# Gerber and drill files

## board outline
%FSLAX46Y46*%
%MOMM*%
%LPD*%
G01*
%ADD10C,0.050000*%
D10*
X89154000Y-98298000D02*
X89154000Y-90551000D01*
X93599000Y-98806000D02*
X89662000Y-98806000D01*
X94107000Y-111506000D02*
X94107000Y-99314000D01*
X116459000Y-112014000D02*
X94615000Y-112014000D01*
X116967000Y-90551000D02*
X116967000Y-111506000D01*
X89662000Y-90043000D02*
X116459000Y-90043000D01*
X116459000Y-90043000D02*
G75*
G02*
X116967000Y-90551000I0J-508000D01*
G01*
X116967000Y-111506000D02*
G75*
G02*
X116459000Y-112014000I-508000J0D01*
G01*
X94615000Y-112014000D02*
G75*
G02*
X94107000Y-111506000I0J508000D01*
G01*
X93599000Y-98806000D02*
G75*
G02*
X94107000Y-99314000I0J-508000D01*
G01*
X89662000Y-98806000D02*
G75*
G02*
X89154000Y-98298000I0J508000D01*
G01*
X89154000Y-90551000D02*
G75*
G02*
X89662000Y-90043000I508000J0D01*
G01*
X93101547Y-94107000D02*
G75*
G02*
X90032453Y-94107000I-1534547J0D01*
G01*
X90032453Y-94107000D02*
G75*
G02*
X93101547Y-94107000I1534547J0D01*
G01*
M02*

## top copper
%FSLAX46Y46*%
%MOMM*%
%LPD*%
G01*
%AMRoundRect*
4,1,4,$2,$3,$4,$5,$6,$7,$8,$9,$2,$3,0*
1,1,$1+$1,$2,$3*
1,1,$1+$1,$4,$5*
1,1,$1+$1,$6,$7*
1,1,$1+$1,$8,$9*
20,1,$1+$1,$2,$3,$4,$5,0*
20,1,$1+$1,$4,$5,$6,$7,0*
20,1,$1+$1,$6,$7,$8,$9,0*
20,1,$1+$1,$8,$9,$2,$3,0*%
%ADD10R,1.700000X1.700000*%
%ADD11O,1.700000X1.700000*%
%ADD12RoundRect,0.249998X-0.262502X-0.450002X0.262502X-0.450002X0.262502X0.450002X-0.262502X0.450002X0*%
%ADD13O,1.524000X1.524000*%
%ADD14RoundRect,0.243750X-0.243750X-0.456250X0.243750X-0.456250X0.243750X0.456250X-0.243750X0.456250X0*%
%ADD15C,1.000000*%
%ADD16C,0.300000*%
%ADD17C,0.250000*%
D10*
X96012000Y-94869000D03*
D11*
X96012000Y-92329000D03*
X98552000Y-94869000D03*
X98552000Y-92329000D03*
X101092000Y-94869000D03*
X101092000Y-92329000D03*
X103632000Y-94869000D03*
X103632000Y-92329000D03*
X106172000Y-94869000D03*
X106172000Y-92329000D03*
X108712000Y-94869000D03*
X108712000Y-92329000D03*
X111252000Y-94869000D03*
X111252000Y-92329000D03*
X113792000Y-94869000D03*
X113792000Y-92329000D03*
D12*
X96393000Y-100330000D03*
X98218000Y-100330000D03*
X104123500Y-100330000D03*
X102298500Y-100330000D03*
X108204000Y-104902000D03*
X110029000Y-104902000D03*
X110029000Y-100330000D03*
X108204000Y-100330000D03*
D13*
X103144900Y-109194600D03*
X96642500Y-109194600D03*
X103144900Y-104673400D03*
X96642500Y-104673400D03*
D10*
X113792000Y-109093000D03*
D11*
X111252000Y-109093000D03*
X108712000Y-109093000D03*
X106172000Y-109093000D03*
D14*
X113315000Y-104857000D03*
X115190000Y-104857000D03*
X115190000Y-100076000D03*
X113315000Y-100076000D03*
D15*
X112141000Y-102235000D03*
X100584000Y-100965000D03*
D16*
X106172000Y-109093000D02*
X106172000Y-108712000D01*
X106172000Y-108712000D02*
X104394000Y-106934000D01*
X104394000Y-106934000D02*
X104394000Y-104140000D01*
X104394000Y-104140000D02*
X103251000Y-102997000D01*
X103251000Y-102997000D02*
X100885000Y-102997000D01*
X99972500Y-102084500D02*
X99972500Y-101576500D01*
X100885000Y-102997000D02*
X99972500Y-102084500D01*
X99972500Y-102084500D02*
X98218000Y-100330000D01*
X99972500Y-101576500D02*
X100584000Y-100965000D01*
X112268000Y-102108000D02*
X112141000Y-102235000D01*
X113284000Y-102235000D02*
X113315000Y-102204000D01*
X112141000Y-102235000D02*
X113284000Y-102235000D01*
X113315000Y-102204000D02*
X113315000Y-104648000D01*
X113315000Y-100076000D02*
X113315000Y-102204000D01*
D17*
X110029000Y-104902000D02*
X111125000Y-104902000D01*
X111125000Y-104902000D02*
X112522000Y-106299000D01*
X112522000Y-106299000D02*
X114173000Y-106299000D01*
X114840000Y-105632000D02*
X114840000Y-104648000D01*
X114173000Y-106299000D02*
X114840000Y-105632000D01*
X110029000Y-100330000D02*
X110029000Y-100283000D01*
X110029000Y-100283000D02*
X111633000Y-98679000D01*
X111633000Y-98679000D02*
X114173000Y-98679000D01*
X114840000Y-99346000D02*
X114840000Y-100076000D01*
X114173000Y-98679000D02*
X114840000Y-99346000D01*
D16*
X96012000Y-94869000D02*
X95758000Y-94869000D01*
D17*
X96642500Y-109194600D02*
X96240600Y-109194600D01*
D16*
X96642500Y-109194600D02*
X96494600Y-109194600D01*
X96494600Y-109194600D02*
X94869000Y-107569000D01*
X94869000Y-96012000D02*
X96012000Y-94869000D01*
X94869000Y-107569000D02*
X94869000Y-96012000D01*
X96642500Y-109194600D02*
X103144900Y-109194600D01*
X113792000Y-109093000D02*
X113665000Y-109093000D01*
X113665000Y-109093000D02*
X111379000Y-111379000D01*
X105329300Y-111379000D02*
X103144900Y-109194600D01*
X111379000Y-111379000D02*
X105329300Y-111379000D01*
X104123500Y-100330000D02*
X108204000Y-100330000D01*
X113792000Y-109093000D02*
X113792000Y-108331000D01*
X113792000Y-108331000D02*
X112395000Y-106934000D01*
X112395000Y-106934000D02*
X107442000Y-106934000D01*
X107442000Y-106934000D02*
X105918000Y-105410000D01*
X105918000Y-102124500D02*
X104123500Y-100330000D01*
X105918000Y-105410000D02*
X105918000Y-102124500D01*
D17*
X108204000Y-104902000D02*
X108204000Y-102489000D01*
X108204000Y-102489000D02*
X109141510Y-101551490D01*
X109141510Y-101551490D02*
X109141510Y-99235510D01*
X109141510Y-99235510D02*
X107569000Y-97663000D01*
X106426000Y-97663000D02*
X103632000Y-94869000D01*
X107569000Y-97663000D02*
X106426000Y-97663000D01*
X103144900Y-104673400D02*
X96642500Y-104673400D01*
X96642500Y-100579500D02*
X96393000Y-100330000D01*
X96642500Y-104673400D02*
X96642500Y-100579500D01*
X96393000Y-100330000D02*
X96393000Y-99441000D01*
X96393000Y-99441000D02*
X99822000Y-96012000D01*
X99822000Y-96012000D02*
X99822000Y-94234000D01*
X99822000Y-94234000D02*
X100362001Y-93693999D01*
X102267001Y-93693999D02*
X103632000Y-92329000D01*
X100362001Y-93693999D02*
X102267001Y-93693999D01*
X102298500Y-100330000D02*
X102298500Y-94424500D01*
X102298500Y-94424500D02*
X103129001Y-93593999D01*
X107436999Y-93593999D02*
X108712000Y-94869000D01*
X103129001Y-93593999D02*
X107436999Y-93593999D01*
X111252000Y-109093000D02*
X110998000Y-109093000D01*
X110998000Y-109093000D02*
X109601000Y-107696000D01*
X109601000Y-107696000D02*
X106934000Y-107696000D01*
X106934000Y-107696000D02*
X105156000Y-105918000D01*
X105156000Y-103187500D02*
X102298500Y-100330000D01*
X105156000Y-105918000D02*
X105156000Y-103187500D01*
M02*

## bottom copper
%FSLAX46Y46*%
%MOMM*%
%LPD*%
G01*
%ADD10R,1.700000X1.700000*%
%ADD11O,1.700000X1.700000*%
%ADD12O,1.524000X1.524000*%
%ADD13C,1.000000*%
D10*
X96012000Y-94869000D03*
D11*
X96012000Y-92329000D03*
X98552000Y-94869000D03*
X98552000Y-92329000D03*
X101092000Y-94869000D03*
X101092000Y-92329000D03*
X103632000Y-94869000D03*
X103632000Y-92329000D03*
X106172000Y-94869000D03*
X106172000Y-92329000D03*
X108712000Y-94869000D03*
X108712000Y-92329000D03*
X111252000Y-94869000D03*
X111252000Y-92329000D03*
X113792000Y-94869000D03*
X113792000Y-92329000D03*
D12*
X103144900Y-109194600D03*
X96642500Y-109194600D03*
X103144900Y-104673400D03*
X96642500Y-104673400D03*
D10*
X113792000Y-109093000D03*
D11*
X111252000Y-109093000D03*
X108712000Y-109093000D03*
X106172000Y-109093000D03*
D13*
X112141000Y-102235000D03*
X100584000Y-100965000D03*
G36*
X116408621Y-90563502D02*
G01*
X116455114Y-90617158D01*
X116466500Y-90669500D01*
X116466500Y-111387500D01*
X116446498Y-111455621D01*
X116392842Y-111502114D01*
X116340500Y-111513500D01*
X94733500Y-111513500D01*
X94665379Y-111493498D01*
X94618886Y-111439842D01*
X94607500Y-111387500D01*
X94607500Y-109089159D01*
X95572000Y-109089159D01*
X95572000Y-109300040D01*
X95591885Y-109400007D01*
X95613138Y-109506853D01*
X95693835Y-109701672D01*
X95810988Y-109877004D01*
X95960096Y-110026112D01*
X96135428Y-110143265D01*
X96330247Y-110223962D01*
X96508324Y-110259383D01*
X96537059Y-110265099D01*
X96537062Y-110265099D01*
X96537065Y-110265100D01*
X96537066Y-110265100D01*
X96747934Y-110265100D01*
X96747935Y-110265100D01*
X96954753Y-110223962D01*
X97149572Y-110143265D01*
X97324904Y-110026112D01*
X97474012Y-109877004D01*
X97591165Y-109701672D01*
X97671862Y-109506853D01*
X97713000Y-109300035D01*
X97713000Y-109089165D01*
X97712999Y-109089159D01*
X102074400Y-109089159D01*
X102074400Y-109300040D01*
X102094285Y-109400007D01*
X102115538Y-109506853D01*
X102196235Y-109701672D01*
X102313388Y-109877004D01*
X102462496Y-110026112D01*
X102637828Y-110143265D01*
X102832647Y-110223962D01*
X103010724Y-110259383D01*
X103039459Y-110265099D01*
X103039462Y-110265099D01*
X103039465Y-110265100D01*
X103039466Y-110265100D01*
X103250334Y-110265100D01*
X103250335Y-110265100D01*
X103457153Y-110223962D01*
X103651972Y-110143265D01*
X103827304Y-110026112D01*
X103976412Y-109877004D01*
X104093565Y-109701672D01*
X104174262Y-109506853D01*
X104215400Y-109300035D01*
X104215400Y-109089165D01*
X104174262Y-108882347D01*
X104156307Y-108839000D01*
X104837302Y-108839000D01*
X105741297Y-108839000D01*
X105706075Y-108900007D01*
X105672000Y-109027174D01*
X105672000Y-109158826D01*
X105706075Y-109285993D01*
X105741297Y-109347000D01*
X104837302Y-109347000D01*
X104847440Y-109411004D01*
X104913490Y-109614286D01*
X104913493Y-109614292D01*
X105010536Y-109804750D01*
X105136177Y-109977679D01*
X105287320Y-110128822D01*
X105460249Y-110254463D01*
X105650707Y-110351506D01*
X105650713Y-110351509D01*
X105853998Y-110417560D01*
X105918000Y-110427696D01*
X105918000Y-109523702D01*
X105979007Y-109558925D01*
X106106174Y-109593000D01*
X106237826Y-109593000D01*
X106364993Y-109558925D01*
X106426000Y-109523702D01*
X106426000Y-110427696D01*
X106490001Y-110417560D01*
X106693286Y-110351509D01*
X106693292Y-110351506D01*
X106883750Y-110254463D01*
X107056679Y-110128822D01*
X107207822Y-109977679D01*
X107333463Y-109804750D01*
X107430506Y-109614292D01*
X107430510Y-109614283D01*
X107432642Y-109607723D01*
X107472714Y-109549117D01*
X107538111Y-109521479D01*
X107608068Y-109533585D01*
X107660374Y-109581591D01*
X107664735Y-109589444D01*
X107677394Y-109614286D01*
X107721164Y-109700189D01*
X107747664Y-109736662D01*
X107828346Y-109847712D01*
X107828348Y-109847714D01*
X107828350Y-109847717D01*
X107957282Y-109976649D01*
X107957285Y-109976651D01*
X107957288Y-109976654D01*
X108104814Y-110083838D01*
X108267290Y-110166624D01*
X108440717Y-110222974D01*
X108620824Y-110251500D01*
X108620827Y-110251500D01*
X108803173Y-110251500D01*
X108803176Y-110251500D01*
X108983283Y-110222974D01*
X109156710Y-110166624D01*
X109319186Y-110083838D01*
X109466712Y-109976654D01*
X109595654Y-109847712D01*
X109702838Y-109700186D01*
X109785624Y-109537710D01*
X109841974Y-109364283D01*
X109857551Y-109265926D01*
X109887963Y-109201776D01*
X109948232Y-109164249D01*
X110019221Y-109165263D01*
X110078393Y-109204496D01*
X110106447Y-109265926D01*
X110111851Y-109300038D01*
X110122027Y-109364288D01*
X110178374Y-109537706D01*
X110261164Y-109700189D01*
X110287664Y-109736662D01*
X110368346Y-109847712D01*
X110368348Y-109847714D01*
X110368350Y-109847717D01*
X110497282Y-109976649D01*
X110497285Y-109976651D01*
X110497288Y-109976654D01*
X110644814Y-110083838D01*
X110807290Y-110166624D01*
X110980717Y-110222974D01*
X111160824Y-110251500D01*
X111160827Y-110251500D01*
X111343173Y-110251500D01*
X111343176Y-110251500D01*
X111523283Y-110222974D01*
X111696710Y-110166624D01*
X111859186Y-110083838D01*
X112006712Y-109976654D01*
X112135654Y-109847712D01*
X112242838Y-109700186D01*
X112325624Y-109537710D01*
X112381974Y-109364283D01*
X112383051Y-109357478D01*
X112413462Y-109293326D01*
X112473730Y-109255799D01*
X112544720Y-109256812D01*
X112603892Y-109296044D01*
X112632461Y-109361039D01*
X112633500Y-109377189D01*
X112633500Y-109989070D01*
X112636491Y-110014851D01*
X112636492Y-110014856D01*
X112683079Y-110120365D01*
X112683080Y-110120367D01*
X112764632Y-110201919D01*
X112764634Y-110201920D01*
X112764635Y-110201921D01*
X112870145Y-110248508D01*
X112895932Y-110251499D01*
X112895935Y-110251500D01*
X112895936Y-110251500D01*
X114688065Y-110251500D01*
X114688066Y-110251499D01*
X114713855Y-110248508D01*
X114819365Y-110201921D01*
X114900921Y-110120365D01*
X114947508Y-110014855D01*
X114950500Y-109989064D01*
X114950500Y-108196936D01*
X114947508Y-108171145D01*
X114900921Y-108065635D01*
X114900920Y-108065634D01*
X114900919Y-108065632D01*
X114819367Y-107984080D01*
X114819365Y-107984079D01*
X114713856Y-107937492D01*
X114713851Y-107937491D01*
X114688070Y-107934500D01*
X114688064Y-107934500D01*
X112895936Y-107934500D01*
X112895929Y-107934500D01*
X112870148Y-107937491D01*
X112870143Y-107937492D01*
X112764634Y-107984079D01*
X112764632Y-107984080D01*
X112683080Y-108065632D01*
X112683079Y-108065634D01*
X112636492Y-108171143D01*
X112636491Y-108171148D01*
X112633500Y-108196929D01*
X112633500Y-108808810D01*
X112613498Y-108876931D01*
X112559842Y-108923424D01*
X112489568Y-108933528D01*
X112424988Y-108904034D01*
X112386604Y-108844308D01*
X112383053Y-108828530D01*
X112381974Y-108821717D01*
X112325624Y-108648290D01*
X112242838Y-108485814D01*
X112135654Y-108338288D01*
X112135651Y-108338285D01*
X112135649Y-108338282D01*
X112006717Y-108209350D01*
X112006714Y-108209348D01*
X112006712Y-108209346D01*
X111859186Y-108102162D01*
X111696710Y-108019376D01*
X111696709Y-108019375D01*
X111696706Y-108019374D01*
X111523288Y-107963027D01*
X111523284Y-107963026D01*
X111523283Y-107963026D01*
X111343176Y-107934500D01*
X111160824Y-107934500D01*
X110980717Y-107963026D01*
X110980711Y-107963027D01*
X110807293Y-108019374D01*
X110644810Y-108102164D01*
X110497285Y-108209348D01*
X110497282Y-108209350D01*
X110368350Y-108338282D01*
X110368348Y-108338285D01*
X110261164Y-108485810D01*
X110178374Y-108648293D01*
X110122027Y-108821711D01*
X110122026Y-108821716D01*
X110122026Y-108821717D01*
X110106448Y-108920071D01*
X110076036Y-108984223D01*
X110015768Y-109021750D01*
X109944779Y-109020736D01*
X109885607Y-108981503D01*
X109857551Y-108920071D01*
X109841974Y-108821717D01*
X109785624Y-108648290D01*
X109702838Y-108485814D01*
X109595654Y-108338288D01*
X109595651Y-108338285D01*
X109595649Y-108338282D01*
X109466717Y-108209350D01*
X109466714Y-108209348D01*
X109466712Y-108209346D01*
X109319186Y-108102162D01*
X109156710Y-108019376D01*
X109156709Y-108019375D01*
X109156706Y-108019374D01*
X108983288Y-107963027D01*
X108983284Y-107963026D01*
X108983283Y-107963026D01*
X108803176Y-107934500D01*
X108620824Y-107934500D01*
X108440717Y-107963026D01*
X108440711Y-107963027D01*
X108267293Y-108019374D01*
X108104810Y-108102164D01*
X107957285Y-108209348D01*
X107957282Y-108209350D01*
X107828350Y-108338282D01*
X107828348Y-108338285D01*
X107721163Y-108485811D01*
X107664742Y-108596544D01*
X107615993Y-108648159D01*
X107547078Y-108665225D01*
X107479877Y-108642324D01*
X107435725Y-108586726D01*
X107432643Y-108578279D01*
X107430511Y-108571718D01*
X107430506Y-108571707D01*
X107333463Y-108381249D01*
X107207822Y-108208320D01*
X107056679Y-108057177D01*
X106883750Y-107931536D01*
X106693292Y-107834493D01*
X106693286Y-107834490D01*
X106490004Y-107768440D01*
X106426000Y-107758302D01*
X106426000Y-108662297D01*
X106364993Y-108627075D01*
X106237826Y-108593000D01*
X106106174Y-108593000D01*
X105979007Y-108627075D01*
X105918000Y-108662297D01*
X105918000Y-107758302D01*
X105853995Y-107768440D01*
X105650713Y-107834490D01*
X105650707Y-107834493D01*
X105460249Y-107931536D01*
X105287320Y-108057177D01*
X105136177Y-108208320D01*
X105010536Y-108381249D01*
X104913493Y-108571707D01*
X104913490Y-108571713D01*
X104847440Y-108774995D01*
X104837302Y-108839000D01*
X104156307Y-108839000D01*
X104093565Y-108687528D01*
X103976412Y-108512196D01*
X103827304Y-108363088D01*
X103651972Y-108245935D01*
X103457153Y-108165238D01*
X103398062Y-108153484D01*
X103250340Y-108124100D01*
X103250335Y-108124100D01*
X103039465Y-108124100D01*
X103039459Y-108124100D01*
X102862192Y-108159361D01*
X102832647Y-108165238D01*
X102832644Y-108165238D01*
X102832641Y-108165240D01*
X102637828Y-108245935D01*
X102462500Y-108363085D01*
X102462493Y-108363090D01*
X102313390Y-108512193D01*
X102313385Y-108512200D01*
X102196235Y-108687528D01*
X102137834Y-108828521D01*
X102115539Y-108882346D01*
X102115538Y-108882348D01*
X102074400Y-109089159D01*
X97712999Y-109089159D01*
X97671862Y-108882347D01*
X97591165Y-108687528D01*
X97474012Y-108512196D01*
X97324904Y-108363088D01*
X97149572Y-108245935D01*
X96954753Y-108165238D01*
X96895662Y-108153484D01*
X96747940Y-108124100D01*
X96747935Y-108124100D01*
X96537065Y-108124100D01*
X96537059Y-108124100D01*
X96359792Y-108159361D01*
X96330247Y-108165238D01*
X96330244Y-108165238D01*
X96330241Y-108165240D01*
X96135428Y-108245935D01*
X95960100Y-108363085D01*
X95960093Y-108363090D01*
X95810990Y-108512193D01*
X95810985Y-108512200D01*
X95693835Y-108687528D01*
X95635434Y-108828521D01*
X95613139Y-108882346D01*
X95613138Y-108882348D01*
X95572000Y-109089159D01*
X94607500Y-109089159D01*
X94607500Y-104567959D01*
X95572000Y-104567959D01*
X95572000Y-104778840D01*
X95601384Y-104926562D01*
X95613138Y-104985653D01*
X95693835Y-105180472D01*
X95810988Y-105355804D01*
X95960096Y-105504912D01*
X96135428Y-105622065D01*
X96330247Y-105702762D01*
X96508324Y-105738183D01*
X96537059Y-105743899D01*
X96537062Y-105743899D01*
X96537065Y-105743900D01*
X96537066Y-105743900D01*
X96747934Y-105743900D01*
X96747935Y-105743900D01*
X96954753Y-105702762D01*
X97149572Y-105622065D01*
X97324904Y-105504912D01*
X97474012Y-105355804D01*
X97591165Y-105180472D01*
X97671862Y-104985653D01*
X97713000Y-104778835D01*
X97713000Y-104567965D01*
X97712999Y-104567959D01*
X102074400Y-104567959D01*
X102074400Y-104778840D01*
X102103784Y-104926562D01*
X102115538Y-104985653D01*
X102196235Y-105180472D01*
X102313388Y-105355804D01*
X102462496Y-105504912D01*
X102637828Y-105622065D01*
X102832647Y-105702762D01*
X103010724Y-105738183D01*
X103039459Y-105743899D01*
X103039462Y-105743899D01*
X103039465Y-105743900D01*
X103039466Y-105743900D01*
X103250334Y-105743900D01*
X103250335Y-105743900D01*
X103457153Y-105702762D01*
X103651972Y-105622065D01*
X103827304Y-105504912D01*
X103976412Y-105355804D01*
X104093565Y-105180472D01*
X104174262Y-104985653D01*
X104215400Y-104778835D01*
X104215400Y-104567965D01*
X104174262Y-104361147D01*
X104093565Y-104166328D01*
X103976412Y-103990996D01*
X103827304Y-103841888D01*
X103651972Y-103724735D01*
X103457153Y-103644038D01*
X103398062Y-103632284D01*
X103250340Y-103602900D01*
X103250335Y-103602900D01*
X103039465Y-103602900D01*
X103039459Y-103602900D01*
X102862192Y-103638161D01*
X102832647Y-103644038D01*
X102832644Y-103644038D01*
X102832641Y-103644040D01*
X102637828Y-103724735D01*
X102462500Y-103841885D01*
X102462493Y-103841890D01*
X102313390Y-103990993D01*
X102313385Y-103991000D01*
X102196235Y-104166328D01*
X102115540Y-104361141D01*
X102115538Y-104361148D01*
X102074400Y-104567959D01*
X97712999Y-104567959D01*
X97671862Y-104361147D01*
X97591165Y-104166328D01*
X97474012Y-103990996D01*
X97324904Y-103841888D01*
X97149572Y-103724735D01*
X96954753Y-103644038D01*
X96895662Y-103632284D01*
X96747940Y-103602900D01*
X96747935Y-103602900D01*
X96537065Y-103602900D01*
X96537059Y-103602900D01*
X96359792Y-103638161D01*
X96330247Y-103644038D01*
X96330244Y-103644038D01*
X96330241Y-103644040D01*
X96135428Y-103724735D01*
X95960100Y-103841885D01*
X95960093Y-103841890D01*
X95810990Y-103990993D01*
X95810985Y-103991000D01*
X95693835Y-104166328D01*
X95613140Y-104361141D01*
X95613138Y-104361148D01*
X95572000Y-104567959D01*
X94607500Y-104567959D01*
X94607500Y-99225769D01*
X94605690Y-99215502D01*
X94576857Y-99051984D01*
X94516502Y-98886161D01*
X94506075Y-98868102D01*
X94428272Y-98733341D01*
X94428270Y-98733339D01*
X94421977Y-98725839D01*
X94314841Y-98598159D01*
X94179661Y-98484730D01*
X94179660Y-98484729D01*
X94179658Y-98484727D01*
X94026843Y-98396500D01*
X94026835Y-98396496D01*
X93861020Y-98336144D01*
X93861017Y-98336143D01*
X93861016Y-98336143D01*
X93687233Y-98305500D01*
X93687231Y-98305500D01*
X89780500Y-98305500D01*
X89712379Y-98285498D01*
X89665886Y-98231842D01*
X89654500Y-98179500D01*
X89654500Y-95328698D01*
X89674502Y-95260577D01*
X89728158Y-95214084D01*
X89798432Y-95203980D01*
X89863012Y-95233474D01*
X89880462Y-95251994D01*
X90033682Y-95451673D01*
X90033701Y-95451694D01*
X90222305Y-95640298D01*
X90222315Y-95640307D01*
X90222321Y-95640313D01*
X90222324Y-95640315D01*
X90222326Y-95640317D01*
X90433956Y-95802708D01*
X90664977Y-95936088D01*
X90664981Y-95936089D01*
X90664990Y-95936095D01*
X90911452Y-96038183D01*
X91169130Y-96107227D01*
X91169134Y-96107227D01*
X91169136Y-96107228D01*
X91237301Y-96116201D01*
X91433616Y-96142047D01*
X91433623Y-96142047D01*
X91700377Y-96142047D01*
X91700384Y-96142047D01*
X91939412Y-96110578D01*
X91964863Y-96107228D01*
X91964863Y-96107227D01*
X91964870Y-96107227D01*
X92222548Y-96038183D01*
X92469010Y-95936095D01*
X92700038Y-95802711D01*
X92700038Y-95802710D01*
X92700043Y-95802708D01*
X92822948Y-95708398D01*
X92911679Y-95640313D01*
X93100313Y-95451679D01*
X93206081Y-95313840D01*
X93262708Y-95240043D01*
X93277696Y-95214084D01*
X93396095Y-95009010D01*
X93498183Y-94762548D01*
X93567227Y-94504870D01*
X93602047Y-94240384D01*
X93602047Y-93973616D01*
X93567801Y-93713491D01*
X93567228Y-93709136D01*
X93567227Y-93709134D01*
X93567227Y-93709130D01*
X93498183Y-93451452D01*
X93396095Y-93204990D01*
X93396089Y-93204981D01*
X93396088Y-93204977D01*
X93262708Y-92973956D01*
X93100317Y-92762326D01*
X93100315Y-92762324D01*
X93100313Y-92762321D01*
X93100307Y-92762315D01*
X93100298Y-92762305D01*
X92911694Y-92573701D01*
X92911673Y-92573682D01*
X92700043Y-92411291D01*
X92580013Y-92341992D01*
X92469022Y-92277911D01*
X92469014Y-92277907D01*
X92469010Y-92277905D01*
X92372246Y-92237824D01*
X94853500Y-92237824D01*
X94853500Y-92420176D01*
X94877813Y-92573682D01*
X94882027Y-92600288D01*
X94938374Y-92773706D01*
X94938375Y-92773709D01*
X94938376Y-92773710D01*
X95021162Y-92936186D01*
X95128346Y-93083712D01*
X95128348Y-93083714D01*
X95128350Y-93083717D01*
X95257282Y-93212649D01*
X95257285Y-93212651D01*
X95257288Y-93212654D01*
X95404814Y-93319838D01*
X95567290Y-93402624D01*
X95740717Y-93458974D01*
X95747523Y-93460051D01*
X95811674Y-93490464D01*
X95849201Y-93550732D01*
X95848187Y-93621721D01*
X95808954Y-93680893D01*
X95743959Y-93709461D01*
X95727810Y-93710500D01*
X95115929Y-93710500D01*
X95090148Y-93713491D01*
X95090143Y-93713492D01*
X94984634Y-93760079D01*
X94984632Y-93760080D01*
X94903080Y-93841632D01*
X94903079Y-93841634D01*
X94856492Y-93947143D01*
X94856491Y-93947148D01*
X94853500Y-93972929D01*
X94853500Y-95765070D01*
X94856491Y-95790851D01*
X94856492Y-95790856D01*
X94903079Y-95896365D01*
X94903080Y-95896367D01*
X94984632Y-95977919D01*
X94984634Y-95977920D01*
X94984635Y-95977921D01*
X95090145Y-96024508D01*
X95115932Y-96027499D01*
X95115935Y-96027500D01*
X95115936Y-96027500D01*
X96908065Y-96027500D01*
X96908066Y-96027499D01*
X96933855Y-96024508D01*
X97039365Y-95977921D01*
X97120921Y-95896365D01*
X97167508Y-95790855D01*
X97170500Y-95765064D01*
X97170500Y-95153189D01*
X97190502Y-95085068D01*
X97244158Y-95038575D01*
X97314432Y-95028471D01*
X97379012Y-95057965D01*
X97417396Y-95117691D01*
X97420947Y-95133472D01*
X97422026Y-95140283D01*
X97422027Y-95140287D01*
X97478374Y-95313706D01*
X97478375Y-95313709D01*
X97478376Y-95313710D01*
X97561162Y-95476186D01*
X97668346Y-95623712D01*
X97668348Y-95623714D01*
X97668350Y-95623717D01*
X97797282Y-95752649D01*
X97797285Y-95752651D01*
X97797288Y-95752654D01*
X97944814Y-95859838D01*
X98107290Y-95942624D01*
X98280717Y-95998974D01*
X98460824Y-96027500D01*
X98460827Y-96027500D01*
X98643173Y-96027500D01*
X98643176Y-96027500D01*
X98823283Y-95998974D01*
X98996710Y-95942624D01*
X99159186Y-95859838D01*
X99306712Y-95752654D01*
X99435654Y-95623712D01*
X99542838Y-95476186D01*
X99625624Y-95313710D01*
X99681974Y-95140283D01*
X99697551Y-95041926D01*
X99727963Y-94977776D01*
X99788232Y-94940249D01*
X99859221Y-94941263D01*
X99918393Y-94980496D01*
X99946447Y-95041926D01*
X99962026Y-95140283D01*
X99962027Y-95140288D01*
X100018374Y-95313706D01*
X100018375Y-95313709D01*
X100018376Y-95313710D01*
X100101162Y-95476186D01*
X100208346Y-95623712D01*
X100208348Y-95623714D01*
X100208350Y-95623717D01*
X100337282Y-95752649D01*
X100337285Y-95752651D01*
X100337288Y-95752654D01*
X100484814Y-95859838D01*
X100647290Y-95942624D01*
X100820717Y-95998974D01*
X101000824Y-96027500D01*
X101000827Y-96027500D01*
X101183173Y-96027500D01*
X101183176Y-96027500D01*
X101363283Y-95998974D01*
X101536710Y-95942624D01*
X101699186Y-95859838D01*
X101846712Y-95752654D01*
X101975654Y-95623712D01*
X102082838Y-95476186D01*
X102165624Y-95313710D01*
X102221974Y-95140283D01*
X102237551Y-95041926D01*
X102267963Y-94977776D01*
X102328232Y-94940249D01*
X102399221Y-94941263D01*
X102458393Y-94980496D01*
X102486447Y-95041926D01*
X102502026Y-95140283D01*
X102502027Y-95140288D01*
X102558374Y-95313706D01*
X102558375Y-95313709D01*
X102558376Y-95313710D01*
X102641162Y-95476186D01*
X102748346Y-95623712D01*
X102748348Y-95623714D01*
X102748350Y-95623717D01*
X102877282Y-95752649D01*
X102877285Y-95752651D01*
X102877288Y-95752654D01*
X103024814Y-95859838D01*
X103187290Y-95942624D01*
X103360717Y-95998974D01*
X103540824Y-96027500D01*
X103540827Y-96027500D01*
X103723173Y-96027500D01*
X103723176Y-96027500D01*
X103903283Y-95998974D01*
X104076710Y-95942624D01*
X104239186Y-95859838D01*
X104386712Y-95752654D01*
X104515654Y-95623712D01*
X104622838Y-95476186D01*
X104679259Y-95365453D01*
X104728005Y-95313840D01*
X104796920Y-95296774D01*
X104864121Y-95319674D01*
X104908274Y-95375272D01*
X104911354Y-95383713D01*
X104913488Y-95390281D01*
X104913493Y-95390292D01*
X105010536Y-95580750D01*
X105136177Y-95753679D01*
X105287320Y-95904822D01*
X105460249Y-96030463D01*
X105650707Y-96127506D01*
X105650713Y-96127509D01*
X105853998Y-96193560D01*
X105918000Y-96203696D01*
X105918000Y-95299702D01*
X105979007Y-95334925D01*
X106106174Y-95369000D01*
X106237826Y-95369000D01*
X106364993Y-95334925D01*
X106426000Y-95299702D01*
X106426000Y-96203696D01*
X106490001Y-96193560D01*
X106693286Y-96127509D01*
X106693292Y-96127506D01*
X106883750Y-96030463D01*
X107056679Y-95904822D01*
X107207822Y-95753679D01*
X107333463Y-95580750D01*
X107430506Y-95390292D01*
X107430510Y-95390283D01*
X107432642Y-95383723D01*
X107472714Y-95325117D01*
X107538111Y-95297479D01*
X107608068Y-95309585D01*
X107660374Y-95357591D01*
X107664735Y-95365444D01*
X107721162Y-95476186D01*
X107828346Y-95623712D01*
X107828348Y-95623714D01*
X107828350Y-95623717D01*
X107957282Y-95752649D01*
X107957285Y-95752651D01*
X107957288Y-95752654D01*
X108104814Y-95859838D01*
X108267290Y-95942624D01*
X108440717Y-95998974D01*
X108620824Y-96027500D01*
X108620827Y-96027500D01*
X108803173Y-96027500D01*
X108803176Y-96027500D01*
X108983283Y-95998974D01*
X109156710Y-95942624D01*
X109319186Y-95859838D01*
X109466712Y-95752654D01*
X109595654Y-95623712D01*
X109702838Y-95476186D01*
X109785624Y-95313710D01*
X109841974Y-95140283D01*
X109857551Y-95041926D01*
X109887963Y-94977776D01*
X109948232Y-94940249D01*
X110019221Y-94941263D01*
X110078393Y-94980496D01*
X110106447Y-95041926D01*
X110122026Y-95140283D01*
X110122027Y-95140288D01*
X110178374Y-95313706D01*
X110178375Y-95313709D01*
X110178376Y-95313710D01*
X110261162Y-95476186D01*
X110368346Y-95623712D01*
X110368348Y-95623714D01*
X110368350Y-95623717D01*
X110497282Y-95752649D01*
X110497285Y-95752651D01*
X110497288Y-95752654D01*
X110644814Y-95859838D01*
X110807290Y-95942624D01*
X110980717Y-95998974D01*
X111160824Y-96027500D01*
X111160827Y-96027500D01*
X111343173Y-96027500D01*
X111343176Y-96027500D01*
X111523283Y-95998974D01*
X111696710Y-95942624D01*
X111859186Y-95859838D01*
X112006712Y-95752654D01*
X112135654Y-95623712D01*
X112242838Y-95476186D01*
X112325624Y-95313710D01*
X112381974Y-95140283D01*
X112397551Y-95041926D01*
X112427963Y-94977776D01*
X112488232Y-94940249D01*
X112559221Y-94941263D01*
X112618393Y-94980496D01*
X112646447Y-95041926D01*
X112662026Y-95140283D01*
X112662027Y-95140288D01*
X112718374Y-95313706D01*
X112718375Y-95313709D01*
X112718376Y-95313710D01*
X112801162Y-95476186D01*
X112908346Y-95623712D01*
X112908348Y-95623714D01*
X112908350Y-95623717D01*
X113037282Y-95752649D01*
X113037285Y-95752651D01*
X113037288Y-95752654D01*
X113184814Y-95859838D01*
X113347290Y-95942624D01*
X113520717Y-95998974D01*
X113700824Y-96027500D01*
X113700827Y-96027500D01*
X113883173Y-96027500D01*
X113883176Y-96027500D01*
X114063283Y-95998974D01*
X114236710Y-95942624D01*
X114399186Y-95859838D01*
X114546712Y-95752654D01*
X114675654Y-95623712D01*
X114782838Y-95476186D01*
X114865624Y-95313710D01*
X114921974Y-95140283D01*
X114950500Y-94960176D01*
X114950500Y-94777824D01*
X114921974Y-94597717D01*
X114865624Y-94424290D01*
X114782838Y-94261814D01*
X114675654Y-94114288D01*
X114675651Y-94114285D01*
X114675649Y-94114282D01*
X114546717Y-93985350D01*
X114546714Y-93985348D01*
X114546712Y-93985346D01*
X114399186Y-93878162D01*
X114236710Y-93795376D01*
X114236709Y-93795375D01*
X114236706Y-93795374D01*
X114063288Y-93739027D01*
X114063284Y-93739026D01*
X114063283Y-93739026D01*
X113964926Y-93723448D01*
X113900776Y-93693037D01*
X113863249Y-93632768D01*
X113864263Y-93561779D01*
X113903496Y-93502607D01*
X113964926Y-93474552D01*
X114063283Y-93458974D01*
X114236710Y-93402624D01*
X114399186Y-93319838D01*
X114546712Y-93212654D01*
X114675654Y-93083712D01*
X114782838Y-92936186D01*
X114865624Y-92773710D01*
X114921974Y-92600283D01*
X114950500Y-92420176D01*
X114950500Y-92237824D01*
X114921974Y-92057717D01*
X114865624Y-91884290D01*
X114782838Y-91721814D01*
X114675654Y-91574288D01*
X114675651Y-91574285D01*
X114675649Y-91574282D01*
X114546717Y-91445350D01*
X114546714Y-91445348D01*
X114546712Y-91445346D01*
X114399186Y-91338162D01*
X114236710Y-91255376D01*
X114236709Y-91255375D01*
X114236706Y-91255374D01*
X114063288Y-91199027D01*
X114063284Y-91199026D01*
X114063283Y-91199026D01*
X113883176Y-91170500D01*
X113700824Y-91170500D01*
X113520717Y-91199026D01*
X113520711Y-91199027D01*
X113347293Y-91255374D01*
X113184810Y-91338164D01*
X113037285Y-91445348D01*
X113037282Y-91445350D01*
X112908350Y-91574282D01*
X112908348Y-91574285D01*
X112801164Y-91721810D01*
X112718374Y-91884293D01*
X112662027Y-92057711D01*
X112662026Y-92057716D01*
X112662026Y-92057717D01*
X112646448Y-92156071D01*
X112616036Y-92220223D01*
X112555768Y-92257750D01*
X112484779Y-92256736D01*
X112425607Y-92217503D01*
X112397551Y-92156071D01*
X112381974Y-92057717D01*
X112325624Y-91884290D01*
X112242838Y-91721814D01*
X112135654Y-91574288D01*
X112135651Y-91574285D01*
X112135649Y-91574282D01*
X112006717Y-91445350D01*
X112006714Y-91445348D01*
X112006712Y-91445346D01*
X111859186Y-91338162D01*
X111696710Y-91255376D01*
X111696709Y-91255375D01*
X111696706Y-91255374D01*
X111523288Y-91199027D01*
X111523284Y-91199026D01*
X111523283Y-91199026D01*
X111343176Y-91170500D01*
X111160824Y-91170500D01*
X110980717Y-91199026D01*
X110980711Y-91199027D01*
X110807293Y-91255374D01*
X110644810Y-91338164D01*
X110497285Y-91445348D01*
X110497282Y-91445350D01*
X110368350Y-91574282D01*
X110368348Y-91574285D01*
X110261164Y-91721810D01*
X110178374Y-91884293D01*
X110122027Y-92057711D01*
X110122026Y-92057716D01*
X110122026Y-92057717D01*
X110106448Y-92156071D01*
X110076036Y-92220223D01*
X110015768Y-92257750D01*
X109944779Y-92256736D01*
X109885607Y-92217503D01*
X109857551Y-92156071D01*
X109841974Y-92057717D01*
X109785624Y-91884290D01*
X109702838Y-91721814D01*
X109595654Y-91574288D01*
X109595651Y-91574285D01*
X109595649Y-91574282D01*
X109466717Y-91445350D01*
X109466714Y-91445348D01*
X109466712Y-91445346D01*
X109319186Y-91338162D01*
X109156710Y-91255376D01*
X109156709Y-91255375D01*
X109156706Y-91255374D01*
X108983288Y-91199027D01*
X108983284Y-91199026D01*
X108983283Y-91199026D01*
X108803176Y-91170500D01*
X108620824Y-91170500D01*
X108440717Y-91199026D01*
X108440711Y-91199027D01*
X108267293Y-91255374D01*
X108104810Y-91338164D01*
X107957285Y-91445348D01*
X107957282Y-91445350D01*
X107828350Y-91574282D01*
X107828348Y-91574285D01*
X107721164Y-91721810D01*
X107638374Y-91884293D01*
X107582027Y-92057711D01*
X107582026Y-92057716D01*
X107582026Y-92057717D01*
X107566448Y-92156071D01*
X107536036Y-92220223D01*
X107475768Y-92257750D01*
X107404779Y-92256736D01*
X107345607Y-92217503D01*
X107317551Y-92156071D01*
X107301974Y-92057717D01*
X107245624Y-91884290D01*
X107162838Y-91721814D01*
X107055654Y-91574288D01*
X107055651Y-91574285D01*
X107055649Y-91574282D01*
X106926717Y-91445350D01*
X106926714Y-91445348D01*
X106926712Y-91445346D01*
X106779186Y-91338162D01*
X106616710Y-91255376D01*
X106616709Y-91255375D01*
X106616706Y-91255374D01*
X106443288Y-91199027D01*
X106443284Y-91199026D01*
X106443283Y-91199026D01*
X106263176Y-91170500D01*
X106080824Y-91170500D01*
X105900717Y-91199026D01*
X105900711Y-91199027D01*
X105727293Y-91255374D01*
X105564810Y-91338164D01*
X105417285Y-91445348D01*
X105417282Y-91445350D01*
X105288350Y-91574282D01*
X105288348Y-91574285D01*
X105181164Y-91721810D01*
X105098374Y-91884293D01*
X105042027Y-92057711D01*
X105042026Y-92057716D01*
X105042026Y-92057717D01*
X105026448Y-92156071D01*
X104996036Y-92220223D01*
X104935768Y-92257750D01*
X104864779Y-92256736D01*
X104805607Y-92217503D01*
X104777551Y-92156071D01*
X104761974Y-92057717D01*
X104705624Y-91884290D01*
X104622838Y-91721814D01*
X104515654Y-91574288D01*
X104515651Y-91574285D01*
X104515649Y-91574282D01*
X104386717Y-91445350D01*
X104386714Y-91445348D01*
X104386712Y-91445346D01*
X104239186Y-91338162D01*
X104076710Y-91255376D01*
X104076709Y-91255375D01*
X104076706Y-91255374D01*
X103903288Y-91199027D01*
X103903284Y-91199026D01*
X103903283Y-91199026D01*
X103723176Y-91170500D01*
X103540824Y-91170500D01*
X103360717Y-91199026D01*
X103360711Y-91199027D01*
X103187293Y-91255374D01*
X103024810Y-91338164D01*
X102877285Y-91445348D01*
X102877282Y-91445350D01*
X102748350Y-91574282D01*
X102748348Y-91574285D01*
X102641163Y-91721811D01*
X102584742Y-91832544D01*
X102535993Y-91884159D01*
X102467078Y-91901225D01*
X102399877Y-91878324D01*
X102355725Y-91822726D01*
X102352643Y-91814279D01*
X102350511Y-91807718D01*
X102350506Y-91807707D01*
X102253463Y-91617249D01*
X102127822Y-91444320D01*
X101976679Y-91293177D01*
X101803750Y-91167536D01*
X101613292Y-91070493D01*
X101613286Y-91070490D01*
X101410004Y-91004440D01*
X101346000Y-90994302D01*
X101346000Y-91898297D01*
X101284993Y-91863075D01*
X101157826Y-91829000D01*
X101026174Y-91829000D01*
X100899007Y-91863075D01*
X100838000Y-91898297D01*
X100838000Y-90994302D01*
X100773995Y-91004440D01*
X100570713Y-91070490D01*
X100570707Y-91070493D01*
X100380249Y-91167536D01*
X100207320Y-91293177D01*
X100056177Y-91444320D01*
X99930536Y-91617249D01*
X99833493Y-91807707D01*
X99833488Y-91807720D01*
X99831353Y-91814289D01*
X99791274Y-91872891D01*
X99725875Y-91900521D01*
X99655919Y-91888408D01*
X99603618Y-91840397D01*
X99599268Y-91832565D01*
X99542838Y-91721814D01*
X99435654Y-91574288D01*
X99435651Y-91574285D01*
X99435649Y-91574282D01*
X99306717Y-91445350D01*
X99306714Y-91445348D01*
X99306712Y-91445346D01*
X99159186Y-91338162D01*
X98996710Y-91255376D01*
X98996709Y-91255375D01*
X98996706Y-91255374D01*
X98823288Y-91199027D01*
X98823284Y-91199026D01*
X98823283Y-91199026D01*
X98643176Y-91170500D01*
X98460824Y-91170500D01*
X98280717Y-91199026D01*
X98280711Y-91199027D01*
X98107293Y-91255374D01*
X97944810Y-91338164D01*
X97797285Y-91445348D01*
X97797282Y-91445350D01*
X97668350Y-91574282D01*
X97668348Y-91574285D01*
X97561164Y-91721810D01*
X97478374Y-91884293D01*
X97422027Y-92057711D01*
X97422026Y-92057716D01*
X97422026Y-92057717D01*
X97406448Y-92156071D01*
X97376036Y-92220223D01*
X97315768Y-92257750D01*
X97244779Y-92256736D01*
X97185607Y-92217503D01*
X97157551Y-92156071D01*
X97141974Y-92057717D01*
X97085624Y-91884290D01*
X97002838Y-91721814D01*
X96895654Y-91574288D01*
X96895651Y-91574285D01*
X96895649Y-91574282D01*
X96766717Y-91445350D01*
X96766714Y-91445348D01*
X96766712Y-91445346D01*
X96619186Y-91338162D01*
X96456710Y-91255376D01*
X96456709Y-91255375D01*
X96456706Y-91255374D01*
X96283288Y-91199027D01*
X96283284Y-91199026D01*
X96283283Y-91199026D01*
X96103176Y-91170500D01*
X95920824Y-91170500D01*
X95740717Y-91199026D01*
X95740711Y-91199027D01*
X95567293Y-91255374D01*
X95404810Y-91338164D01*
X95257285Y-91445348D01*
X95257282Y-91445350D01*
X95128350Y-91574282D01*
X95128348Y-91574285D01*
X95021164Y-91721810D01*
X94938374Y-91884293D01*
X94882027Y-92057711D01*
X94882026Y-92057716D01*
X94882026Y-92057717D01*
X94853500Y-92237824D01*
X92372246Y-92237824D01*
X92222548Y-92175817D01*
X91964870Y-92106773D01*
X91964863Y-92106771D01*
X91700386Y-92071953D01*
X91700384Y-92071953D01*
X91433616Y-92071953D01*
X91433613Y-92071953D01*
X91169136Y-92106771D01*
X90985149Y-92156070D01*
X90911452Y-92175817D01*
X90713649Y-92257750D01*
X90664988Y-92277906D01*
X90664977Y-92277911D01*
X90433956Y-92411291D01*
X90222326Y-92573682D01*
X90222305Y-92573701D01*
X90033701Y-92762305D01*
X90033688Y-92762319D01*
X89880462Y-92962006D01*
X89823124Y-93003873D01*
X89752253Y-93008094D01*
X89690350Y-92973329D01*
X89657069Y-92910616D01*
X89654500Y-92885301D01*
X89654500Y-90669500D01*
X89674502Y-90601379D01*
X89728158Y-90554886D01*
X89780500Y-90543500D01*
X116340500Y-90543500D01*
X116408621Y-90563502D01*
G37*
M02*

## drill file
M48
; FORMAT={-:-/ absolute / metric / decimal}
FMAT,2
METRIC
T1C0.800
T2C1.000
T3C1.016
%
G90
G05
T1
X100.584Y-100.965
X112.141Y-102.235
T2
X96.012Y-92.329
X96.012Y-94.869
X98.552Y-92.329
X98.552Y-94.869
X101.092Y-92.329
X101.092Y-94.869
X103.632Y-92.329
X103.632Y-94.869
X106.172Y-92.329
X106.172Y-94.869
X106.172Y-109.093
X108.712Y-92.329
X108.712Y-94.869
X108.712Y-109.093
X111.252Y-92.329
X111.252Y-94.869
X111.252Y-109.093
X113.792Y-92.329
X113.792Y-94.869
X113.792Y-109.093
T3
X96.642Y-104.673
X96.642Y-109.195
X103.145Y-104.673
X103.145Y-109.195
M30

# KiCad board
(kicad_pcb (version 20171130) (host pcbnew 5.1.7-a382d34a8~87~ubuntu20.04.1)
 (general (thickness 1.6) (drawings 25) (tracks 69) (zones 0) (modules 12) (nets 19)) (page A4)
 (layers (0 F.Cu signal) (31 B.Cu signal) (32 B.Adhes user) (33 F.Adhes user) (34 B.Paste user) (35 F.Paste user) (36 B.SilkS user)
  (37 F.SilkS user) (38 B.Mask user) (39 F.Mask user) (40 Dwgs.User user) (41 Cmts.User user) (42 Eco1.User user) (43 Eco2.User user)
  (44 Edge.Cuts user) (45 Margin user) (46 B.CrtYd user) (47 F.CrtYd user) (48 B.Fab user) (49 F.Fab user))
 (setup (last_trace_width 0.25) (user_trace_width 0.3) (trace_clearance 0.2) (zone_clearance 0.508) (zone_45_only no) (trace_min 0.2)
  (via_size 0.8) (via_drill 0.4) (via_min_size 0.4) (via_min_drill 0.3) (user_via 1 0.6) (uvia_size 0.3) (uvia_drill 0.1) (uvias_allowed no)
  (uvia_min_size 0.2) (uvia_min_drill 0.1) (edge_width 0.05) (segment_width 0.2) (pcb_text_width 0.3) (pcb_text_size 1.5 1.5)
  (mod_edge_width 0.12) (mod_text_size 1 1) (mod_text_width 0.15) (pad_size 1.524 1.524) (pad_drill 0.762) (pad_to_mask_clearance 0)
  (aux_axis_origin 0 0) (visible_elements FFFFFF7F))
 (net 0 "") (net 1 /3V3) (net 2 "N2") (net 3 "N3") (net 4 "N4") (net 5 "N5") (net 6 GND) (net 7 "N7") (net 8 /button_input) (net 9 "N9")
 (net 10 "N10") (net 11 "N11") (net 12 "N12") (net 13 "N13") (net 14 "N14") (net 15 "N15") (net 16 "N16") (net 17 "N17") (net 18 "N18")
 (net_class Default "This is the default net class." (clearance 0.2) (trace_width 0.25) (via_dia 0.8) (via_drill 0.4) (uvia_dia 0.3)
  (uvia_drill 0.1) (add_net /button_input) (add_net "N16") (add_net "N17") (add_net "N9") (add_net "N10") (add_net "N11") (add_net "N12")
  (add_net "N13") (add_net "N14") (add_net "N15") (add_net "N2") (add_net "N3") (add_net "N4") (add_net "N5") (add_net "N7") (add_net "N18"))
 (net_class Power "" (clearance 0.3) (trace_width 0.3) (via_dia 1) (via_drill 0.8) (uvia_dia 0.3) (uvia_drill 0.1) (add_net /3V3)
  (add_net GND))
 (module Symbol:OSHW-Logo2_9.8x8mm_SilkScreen (layer B.Cu) (at 99.568 107.315 180)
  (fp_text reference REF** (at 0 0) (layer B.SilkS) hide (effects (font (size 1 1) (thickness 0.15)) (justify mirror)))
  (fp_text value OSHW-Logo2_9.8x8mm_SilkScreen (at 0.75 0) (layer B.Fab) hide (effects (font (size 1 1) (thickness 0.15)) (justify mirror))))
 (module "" (layer F.Cu) (at 96.012 106.553)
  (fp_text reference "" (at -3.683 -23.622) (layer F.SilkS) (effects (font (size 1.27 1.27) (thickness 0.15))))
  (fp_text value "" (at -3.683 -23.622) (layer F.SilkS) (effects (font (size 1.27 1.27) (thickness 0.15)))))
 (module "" (layer F.Cu) (at -3.683 -23.622)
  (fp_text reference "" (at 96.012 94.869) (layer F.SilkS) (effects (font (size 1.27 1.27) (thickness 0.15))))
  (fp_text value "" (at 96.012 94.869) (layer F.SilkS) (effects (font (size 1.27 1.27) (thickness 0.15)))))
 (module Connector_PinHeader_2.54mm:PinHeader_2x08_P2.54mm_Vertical (layer F.Cu) (at 96.012 94.869 90)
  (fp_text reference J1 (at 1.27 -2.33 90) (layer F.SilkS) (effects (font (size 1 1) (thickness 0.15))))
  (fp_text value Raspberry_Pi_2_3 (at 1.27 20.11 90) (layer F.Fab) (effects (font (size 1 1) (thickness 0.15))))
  (pad 1 thru_hole rect (at 0 0 90) (size 1.7 1.7) (drill 1) (layers *.Cu *.Mask) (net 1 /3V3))
  (pad 2 thru_hole oval (at 2.54 0 90) (size 1.7 1.7) (drill 1) (layers *.Cu *.Mask) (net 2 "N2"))
  (pad 3 thru_hole oval (at 0 2.54 90) (size 1.7 1.7) (drill 1) (layers *.Cu *.Mask) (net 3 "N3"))
  (pad 4 thru_hole oval (at 2.54 2.54 90) (size 1.7 1.7) (drill 1) (layers *.Cu *.Mask) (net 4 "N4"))
  (pad 5 thru_hole oval (at 0 5.08 90) (size 1.7 1.7) (drill 1) (layers *.Cu *.Mask) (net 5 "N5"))
  (pad 6 thru_hole oval (at 2.54 5.08 90) (size 1.7 1.7) (drill 1) (layers *.Cu *.Mask) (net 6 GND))
  (pad 7 thru_hole oval (at 0 7.62 90) (size 1.7 1.7) (drill 1) (layers *.Cu *.Mask) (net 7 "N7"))
  (pad 8 thru_hole oval (at 2.54 7.62 90) (size 1.7 1.7) (drill 1) (layers *.Cu *.Mask) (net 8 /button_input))
  (pad 9 thru_hole oval (at 0 10.16 90) (size 1.7 1.7) (drill 1) (layers *.Cu *.Mask) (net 6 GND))
  (pad 10 thru_hole oval (at 2.54 10.16 90) (size 1.7 1.7) (drill 1) (layers *.Cu *.Mask) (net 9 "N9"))
  (pad 11 thru_hole oval (at 0 12.7 90) (size 1.7 1.7) (drill 1) (layers *.Cu *.Mask) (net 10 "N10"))
  (pad 12 thru_hole oval (at 2.54 12.7 90) (size 1.7 1.7) (drill 1) (layers *.Cu *.Mask) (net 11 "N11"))
  (pad 13 thru_hole oval (at 0 15.24 90) (size 1.7 1.7) (drill 1) (layers *.Cu *.Mask) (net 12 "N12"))
  (pad 14 thru_hole oval (at 2.54 15.24 90) (size 1.7 1.7) (drill 1) (layers *.Cu *.Mask) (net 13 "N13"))
  (pad 15 thru_hole oval (at 0 17.78 90) (size 1.7 1.7) (drill 1) (layers *.Cu *.Mask) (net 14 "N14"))
  (pad 16 thru_hole oval (at 2.54 17.78 90) (size 1.7 1.7) (drill 1) (layers *.Cu *.Mask) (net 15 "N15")))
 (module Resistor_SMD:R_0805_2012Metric (layer F.Cu) (at 97.3055 100.33)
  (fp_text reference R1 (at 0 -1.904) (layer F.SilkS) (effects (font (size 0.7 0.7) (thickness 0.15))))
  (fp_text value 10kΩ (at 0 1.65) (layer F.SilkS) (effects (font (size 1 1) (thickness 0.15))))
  (pad 1 smd roundrect (at -0.9125 0) (size 1.025 1.4) (layers F.Cu F.Paste F.Mask) (roundrect_rratio 0.2439004878048781)
   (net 8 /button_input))
  (pad 2 smd roundrect (at 0.9125 0) (size 1.025 1.4) (layers F.Cu F.Paste F.Mask) (roundrect_rratio 0.2439004878048781) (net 6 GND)))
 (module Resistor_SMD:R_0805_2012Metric (layer F.Cu) (at 103.211 100.33)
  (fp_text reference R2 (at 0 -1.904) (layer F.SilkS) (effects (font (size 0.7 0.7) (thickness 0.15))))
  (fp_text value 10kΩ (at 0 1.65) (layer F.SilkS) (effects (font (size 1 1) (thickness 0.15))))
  (pad 2 smd roundrect (at 0.9125 0) (size 1.025 1.4) (layers F.Cu F.Paste F.Mask) (roundrect_rratio 0.2439004878048781) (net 1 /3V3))
  (pad 1 smd roundrect (at -0.9125 0) (size 1.025 1.4) (layers F.Cu F.Paste F.Mask) (roundrect_rratio 0.2439004878048781) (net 10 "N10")))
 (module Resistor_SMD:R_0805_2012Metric (layer F.Cu) (at 109.1165 104.902)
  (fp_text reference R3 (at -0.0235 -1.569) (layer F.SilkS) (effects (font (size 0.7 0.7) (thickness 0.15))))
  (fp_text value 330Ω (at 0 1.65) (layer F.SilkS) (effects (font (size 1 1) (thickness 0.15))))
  (pad 1 smd roundrect (at -0.9125 0) (size 1.025 1.4) (layers F.Cu F.Paste F.Mask) (roundrect_rratio 0.2439004878048781) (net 7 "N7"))
  (pad 2 smd roundrect (at 0.9125 0) (size 1.025 1.4) (layers F.Cu F.Paste F.Mask) (roundrect_rratio 0.2439004878048781) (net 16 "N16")))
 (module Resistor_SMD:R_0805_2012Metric (layer F.Cu) (at 109.1165 100.33)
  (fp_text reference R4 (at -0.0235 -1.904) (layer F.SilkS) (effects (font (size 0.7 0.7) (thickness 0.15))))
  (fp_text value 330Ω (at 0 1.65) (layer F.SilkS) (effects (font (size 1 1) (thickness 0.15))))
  (pad 2 smd roundrect (at 0.9125 0) (size 1.025 1.4) (layers F.Cu F.Paste F.Mask) (roundrect_rratio 0.2439004878048781) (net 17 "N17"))
  (pad 1 smd roundrect (at -0.9125 0) (size 1.025 1.4) (layers F.Cu F.Paste F.Mask) (roundrect_rratio 0.2439004878048781) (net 1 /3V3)))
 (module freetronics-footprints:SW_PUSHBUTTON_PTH (layer F.Cu) (at 99.8937 106.934 180)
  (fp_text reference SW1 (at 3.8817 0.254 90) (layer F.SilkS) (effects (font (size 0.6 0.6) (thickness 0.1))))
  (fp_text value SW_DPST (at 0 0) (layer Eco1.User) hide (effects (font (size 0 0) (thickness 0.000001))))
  (pad 1 thru_hole oval (at -3.2512 -2.2606 180) (size 1.524 1.524) (drill 1.016) (layers *.Cu *.Mask) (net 1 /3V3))
  (pad 1 thru_hole oval (at 3.2512 -2.2606 180) (size 1.524 1.524) (drill 1.016) (layers *.Cu *.Mask) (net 1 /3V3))
  (pad 2 thru_hole oval (at -3.2512 2.2606 180) (size 1.524 1.524) (drill 1.016) (layers *.Cu *.Mask) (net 8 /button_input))
  (pad 2 thru_hole oval (at 3.2512 2.2606 180) (size 1.524 1.524) (drill 1.016) (layers *.Cu *.Mask) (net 8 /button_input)))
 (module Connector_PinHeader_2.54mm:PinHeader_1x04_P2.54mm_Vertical (layer F.Cu) (at 113.792 109.093 270)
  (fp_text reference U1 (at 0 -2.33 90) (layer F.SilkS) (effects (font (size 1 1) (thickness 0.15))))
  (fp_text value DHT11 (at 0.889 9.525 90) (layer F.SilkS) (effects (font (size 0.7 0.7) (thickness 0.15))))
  (pad 1 thru_hole rect (at 0 0 270) (size 1.7 1.7) (drill 1) (layers *.Cu *.Mask) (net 1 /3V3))
  (pad 2 thru_hole oval (at 0 2.54 270) (size 1.7 1.7) (drill 1) (layers *.Cu *.Mask) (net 10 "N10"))
  (pad 3 thru_hole oval (at 0 5.08 270) (size 1.7 1.7) (drill 1) (layers *.Cu *.Mask) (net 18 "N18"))
  (pad 4 thru_hole oval (at 0 7.62 270) (size 1.7 1.7) (drill 1) (layers *.Cu *.Mask) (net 6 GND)))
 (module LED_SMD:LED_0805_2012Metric (layer F.Cu) (at 114.2525 104.857)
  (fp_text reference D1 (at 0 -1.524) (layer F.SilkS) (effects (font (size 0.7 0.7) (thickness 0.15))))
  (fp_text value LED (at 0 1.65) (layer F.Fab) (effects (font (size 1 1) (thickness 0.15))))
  (pad 1 smd roundrect (at -0.9375 0) (size 0.975 1.4) (layers F.Cu F.Paste F.Mask) (roundrect_rratio 0.25) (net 6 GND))
  (pad 2 smd roundrect (at 0.9375 0) (size 0.975 1.4) (layers F.Cu F.Paste F.Mask) (roundrect_rratio 0.25) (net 16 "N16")))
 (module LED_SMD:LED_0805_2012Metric (layer F.Cu) (at 114.2525 100.076)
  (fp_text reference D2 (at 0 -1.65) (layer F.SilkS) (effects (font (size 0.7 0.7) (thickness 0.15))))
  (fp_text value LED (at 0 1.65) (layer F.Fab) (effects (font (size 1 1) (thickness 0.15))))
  (pad 2 smd roundrect (at 0.9375 0) (size 0.975 1.4) (layers F.Cu F.Paste F.Mask) (roundrect_rratio 0.25) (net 17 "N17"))
  (pad 1 smd roundrect (at -0.9375 0) (size 0.975 1.4) (layers F.Cu F.Paste F.Mask) (roundrect_rratio 0.25) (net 6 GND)))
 (gr_line (start 89.154 98.298) (end 89.154 90.551) (layer Edge.Cuts) (width 0.05))
 (gr_line (start 93.599 98.806) (end 89.662 98.806) (layer Edge.Cuts) (width 0.05))
 (gr_line (start 94.107 111.506) (end 94.107 99.314) (layer Edge.Cuts) (width 0.05))
 (gr_line (start 116.459 112.014) (end 94.615 112.014) (layer Edge.Cuts) (width 0.05))
 (gr_line (start 116.967 90.551) (end 116.967 111.506) (layer Edge.Cuts) (width 0.05))
 (gr_line (start 89.662 90.043) (end 116.459 90.043) (layer Edge.Cuts) (width 0.05))
 (gr_arc (start 116.459 90.551) (end 116.967 90.551) (angle -90) (layer Edge.Cuts) (width 0.05))
 (gr_arc (start 116.459 111.506) (end 116.459 112.014) (angle -90) (layer Edge.Cuts) (width 0.05))
 (gr_arc (start 94.615 111.506) (end 94.107 111.506) (angle -90) (layer Edge.Cuts) (width 0.05))
 (gr_arc (start 93.599 99.314) (end 94.107 99.314) (angle -90) (layer Edge.Cuts) (width 0.05))
 (gr_arc (start 89.662 98.298) (end 89.154 98.298) (angle -90) (layer Edge.Cuts) (width 0.05))
 (gr_arc (start 89.662 90.551) (end 89.662 90.043) (angle -90) (layer Edge.Cuts) (width 0.05))
 (gr_circle (center 91.567 94.107) (end 90.17 93.472) (layer Edge.Cuts) (width 0.05))
 (via (at 112.141 102.235) (size 1) (drill 0.8) (layers F.Cu B.Cu) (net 6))
 (via (at 100.584 100.965) (size 1) (drill 0.8) (layers F.Cu B.Cu) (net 6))
 (segment (start 106.172 109.093) (end 106.172 108.712) (width 0.3) (layer F.Cu) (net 6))
 (segment (start 106.172 108.712) (end 104.394 106.934) (width 0.3) (layer F.Cu) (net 6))
 (segment (start 104.394 106.934) (end 104.394 104.14) (width 0.3) (layer F.Cu) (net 6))
 (segment (start 104.394 104.14) (end 103.251 102.997) (width 0.3) (layer F.Cu) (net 6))
 (segment (start 103.251 102.997) (end 100.885 102.997) (width 0.3) (layer F.Cu) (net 6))
 (segment (start 99.9725 102.0845) (end 99.9725 101.5765) (width 0.3) (layer F.Cu) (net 6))
 (segment (start 100.885 102.997) (end 99.9725 102.0845) (width 0.3) (layer F.Cu) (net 6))
 (segment (start 99.9725 102.0845) (end 98.218 100.33) (width 0.3) (layer F.Cu) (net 6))
 (segment (start 99.9725 101.5765) (end 100.584 100.965) (width 0.3) (layer F.Cu) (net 6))
 (segment (start 112.268 102.108) (end 112.141 102.235) (width 0.3) (layer F.Cu) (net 6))
 (segment (start 113.284 102.235) (end 113.315 102.204) (width 0.3) (layer F.Cu) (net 6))
 (segment (start 112.141 102.235) (end 113.284 102.235) (width 0.3) (layer F.Cu) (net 6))
 (segment (start 113.315 102.204) (end 113.315 104.648) (width 0.3) (layer F.Cu) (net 6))
 (segment (start 113.315 100.076) (end 113.315 102.204) (width 0.3) (layer F.Cu) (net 6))
 (segment (start 110.029 104.902) (end 111.125 104.902) (width 0.25) (layer F.Cu) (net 16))
 (segment (start 111.125 104.902) (end 112.522 106.299) (width 0.25) (layer F.Cu) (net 16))
 (segment (start 112.522 106.299) (end 114.173 106.299) (width 0.25) (layer F.Cu) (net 16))
 (segment (start 114.84 105.632) (end 114.84 104.648) (width 0.25) (layer F.Cu) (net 16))
 (segment (start 114.173 106.299) (end 114.84 105.632) (width 0.25) (layer F.Cu) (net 16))
 (segment (start 110.029 100.33) (end 110.029 100.283) (width 0.25) (layer F.Cu) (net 17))
 (segment (start 110.029 100.283) (end 111.633 98.679) (width 0.25) (layer F.Cu) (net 17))
 (segment (start 111.633 98.679) (end 114.173 98.679) (width 0.25) (layer F.Cu) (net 17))
 (segment (start 114.84 99.346) (end 114.84 100.076) (width 0.25) (layer F.Cu) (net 17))
 (segment (start 114.173 98.679) (end 114.84 99.346) (width 0.25) (layer F.Cu) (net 17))
 (segment (start 96.012 94.869) (end 95.758 94.869) (width 0.3) (layer F.Cu) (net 1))
 (segment (start 96.6425 109.1946) (end 96.2406 109.1946) (width 0.25) (layer F.Cu) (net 1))
 (segment (start 96.6425 109.1946) (end 96.4946 109.1946) (width 0.3) (layer F.Cu) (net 1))
 (segment (start 96.4946 109.1946) (end 94.869 107.569) (width 0.3) (layer F.Cu) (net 1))
 (segment (start 94.869 96.012) (end 96.012 94.869) (width 0.3) (layer F.Cu) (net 1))
 (segment (start 94.869 107.569) (end 94.869 96.012) (width 0.3) (layer F.Cu) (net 1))
 (segment (start 96.6425 109.1946) (end 103.1449 109.1946) (width 0.3) (layer F.Cu) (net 1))
 (segment (start 113.792 109.093) (end 113.665 109.093) (width 0.3) (layer F.Cu) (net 1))
 (segment (start 113.665 109.093) (end 111.379 111.379) (width 0.3) (layer F.Cu) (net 1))
 (segment (start 105.3293 111.379) (end 103.1449 109.1946) (width 0.3) (layer F.Cu) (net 1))
 (segment (start 111.379 111.379) (end 105.3293 111.379) (width 0.3) (layer F.Cu) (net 1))
 (segment (start 104.1235 100.33) (end 108.204 100.33) (width 0.3) (layer F.Cu) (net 1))
 (segment (start 113.792 109.093) (end 113.792 108.331) (width 0.3) (layer F.Cu) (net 1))
 (segment (start 113.792 108.331) (end 112.395 106.934) (width 0.3) (layer F.Cu) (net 1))
 (segment (start 112.395 106.934) (end 107.442 106.934) (width 0.3) (layer F.Cu) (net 1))
 (segment (start 107.442 106.934) (end 105.918 105.41) (width 0.3) (layer F.Cu) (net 1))
 (segment (start 105.918 102.1245) (end 104.1235 100.33) (width 0.3) (layer F.Cu) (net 1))
 (segment (start 105.918 105.41) (end 105.918 102.1245) (width 0.3) (layer F.Cu) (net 1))
 (segment (start 108.204 104.902) (end 108.204 102.489) (width 0.25) (layer F.Cu) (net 7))
 (segment (start 108.204 102.489) (end 109.14151 101.55149) (width 0.25) (layer F.Cu) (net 7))
 (segment (start 109.14151 101.55149) (end 109.14151 99.23551) (width 0.25) (layer F.Cu) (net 7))
 (segment (start 109.14151 99.23551) (end 107.569 97.663) (width 0.25) (layer F.Cu) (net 7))
 (segment (start 106.426 97.663) (end 103.632 94.869) (width 0.25) (layer F.Cu) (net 7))
 (segment (start 107.569 97.663) (end 106.426 97.663) (width 0.25) (layer F.Cu) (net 7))
 (segment (start 103.1449 104.6734) (end 96.6425 104.6734) (width 0.25) (layer F.Cu) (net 8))
 (segment (start 96.6425 100.5795) (end 96.393 100.33) (width 0.25) (layer F.Cu) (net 8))
 (segment (start 96.6425 104.6734) (end 96.6425 100.5795) (width 0.25) (layer F.Cu) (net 8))
 (segment (start 96.393 100.33) (end 96.393 99.441) (width 0.25) (layer F.Cu) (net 8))
 (segment (start 96.393 99.441) (end 99.822 96.012) (width 0.25) (layer F.Cu) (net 8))
 (segment (start 99.822 96.012) (end 99.822 94.234) (width 0.25) (layer F.Cu) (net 8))
 (segment (start 99.822 94.234) (end 100.362001 93.693999) (width 0.25) (layer F.Cu) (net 8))
 (segment (start 102.267001 93.693999) (end 103.632 92.329) (width 0.25) (layer F.Cu) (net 8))
 (segment (start 100.362001 93.693999) (end 102.267001 93.693999) (width 0.25) (layer F.Cu) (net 8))
 (segment (start 102.2985 100.33) (end 102.2985 94.4245) (width 0.25) (layer F.Cu) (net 10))
 (segment (start 102.2985 94.4245) (end 103.129001 93.593999) (width 0.25) (layer F.Cu) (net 10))
 (segment (start 107.436999 93.593999) (end 108.712 94.869) (width 0.25) (layer F.Cu) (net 10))
 (segment (start 103.129001 93.593999) (end 107.436999 93.593999) (width 0.25) (layer F.Cu) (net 10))
 (segment (start 111.252 109.093) (end 110.998 109.093) (width 0.25) (layer F.Cu) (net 10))
 (segment (start 110.998 109.093) (end 109.601 107.696) (width 0.25) (layer F.Cu) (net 10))
 (segment (start 109.601 107.696) (end 106.934 107.696) (width 0.25) (layer F.Cu) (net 10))
 (segment (start 106.934 107.696) (end 105.156 105.918) (width 0.25) (layer F.Cu) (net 10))
 (segment (start 105.156 103.1875) (end 102.2985 100.33) (width 0.25) (layer F.Cu) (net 10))
 (segment (start 105.156 105.918) (end 105.156 103.1875) (width 0.25) (layer F.Cu) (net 10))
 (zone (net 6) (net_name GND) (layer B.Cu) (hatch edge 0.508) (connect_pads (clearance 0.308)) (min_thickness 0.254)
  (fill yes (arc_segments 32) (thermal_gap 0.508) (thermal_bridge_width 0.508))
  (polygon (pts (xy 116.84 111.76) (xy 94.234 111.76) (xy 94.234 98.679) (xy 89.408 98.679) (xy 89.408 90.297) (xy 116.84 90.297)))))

